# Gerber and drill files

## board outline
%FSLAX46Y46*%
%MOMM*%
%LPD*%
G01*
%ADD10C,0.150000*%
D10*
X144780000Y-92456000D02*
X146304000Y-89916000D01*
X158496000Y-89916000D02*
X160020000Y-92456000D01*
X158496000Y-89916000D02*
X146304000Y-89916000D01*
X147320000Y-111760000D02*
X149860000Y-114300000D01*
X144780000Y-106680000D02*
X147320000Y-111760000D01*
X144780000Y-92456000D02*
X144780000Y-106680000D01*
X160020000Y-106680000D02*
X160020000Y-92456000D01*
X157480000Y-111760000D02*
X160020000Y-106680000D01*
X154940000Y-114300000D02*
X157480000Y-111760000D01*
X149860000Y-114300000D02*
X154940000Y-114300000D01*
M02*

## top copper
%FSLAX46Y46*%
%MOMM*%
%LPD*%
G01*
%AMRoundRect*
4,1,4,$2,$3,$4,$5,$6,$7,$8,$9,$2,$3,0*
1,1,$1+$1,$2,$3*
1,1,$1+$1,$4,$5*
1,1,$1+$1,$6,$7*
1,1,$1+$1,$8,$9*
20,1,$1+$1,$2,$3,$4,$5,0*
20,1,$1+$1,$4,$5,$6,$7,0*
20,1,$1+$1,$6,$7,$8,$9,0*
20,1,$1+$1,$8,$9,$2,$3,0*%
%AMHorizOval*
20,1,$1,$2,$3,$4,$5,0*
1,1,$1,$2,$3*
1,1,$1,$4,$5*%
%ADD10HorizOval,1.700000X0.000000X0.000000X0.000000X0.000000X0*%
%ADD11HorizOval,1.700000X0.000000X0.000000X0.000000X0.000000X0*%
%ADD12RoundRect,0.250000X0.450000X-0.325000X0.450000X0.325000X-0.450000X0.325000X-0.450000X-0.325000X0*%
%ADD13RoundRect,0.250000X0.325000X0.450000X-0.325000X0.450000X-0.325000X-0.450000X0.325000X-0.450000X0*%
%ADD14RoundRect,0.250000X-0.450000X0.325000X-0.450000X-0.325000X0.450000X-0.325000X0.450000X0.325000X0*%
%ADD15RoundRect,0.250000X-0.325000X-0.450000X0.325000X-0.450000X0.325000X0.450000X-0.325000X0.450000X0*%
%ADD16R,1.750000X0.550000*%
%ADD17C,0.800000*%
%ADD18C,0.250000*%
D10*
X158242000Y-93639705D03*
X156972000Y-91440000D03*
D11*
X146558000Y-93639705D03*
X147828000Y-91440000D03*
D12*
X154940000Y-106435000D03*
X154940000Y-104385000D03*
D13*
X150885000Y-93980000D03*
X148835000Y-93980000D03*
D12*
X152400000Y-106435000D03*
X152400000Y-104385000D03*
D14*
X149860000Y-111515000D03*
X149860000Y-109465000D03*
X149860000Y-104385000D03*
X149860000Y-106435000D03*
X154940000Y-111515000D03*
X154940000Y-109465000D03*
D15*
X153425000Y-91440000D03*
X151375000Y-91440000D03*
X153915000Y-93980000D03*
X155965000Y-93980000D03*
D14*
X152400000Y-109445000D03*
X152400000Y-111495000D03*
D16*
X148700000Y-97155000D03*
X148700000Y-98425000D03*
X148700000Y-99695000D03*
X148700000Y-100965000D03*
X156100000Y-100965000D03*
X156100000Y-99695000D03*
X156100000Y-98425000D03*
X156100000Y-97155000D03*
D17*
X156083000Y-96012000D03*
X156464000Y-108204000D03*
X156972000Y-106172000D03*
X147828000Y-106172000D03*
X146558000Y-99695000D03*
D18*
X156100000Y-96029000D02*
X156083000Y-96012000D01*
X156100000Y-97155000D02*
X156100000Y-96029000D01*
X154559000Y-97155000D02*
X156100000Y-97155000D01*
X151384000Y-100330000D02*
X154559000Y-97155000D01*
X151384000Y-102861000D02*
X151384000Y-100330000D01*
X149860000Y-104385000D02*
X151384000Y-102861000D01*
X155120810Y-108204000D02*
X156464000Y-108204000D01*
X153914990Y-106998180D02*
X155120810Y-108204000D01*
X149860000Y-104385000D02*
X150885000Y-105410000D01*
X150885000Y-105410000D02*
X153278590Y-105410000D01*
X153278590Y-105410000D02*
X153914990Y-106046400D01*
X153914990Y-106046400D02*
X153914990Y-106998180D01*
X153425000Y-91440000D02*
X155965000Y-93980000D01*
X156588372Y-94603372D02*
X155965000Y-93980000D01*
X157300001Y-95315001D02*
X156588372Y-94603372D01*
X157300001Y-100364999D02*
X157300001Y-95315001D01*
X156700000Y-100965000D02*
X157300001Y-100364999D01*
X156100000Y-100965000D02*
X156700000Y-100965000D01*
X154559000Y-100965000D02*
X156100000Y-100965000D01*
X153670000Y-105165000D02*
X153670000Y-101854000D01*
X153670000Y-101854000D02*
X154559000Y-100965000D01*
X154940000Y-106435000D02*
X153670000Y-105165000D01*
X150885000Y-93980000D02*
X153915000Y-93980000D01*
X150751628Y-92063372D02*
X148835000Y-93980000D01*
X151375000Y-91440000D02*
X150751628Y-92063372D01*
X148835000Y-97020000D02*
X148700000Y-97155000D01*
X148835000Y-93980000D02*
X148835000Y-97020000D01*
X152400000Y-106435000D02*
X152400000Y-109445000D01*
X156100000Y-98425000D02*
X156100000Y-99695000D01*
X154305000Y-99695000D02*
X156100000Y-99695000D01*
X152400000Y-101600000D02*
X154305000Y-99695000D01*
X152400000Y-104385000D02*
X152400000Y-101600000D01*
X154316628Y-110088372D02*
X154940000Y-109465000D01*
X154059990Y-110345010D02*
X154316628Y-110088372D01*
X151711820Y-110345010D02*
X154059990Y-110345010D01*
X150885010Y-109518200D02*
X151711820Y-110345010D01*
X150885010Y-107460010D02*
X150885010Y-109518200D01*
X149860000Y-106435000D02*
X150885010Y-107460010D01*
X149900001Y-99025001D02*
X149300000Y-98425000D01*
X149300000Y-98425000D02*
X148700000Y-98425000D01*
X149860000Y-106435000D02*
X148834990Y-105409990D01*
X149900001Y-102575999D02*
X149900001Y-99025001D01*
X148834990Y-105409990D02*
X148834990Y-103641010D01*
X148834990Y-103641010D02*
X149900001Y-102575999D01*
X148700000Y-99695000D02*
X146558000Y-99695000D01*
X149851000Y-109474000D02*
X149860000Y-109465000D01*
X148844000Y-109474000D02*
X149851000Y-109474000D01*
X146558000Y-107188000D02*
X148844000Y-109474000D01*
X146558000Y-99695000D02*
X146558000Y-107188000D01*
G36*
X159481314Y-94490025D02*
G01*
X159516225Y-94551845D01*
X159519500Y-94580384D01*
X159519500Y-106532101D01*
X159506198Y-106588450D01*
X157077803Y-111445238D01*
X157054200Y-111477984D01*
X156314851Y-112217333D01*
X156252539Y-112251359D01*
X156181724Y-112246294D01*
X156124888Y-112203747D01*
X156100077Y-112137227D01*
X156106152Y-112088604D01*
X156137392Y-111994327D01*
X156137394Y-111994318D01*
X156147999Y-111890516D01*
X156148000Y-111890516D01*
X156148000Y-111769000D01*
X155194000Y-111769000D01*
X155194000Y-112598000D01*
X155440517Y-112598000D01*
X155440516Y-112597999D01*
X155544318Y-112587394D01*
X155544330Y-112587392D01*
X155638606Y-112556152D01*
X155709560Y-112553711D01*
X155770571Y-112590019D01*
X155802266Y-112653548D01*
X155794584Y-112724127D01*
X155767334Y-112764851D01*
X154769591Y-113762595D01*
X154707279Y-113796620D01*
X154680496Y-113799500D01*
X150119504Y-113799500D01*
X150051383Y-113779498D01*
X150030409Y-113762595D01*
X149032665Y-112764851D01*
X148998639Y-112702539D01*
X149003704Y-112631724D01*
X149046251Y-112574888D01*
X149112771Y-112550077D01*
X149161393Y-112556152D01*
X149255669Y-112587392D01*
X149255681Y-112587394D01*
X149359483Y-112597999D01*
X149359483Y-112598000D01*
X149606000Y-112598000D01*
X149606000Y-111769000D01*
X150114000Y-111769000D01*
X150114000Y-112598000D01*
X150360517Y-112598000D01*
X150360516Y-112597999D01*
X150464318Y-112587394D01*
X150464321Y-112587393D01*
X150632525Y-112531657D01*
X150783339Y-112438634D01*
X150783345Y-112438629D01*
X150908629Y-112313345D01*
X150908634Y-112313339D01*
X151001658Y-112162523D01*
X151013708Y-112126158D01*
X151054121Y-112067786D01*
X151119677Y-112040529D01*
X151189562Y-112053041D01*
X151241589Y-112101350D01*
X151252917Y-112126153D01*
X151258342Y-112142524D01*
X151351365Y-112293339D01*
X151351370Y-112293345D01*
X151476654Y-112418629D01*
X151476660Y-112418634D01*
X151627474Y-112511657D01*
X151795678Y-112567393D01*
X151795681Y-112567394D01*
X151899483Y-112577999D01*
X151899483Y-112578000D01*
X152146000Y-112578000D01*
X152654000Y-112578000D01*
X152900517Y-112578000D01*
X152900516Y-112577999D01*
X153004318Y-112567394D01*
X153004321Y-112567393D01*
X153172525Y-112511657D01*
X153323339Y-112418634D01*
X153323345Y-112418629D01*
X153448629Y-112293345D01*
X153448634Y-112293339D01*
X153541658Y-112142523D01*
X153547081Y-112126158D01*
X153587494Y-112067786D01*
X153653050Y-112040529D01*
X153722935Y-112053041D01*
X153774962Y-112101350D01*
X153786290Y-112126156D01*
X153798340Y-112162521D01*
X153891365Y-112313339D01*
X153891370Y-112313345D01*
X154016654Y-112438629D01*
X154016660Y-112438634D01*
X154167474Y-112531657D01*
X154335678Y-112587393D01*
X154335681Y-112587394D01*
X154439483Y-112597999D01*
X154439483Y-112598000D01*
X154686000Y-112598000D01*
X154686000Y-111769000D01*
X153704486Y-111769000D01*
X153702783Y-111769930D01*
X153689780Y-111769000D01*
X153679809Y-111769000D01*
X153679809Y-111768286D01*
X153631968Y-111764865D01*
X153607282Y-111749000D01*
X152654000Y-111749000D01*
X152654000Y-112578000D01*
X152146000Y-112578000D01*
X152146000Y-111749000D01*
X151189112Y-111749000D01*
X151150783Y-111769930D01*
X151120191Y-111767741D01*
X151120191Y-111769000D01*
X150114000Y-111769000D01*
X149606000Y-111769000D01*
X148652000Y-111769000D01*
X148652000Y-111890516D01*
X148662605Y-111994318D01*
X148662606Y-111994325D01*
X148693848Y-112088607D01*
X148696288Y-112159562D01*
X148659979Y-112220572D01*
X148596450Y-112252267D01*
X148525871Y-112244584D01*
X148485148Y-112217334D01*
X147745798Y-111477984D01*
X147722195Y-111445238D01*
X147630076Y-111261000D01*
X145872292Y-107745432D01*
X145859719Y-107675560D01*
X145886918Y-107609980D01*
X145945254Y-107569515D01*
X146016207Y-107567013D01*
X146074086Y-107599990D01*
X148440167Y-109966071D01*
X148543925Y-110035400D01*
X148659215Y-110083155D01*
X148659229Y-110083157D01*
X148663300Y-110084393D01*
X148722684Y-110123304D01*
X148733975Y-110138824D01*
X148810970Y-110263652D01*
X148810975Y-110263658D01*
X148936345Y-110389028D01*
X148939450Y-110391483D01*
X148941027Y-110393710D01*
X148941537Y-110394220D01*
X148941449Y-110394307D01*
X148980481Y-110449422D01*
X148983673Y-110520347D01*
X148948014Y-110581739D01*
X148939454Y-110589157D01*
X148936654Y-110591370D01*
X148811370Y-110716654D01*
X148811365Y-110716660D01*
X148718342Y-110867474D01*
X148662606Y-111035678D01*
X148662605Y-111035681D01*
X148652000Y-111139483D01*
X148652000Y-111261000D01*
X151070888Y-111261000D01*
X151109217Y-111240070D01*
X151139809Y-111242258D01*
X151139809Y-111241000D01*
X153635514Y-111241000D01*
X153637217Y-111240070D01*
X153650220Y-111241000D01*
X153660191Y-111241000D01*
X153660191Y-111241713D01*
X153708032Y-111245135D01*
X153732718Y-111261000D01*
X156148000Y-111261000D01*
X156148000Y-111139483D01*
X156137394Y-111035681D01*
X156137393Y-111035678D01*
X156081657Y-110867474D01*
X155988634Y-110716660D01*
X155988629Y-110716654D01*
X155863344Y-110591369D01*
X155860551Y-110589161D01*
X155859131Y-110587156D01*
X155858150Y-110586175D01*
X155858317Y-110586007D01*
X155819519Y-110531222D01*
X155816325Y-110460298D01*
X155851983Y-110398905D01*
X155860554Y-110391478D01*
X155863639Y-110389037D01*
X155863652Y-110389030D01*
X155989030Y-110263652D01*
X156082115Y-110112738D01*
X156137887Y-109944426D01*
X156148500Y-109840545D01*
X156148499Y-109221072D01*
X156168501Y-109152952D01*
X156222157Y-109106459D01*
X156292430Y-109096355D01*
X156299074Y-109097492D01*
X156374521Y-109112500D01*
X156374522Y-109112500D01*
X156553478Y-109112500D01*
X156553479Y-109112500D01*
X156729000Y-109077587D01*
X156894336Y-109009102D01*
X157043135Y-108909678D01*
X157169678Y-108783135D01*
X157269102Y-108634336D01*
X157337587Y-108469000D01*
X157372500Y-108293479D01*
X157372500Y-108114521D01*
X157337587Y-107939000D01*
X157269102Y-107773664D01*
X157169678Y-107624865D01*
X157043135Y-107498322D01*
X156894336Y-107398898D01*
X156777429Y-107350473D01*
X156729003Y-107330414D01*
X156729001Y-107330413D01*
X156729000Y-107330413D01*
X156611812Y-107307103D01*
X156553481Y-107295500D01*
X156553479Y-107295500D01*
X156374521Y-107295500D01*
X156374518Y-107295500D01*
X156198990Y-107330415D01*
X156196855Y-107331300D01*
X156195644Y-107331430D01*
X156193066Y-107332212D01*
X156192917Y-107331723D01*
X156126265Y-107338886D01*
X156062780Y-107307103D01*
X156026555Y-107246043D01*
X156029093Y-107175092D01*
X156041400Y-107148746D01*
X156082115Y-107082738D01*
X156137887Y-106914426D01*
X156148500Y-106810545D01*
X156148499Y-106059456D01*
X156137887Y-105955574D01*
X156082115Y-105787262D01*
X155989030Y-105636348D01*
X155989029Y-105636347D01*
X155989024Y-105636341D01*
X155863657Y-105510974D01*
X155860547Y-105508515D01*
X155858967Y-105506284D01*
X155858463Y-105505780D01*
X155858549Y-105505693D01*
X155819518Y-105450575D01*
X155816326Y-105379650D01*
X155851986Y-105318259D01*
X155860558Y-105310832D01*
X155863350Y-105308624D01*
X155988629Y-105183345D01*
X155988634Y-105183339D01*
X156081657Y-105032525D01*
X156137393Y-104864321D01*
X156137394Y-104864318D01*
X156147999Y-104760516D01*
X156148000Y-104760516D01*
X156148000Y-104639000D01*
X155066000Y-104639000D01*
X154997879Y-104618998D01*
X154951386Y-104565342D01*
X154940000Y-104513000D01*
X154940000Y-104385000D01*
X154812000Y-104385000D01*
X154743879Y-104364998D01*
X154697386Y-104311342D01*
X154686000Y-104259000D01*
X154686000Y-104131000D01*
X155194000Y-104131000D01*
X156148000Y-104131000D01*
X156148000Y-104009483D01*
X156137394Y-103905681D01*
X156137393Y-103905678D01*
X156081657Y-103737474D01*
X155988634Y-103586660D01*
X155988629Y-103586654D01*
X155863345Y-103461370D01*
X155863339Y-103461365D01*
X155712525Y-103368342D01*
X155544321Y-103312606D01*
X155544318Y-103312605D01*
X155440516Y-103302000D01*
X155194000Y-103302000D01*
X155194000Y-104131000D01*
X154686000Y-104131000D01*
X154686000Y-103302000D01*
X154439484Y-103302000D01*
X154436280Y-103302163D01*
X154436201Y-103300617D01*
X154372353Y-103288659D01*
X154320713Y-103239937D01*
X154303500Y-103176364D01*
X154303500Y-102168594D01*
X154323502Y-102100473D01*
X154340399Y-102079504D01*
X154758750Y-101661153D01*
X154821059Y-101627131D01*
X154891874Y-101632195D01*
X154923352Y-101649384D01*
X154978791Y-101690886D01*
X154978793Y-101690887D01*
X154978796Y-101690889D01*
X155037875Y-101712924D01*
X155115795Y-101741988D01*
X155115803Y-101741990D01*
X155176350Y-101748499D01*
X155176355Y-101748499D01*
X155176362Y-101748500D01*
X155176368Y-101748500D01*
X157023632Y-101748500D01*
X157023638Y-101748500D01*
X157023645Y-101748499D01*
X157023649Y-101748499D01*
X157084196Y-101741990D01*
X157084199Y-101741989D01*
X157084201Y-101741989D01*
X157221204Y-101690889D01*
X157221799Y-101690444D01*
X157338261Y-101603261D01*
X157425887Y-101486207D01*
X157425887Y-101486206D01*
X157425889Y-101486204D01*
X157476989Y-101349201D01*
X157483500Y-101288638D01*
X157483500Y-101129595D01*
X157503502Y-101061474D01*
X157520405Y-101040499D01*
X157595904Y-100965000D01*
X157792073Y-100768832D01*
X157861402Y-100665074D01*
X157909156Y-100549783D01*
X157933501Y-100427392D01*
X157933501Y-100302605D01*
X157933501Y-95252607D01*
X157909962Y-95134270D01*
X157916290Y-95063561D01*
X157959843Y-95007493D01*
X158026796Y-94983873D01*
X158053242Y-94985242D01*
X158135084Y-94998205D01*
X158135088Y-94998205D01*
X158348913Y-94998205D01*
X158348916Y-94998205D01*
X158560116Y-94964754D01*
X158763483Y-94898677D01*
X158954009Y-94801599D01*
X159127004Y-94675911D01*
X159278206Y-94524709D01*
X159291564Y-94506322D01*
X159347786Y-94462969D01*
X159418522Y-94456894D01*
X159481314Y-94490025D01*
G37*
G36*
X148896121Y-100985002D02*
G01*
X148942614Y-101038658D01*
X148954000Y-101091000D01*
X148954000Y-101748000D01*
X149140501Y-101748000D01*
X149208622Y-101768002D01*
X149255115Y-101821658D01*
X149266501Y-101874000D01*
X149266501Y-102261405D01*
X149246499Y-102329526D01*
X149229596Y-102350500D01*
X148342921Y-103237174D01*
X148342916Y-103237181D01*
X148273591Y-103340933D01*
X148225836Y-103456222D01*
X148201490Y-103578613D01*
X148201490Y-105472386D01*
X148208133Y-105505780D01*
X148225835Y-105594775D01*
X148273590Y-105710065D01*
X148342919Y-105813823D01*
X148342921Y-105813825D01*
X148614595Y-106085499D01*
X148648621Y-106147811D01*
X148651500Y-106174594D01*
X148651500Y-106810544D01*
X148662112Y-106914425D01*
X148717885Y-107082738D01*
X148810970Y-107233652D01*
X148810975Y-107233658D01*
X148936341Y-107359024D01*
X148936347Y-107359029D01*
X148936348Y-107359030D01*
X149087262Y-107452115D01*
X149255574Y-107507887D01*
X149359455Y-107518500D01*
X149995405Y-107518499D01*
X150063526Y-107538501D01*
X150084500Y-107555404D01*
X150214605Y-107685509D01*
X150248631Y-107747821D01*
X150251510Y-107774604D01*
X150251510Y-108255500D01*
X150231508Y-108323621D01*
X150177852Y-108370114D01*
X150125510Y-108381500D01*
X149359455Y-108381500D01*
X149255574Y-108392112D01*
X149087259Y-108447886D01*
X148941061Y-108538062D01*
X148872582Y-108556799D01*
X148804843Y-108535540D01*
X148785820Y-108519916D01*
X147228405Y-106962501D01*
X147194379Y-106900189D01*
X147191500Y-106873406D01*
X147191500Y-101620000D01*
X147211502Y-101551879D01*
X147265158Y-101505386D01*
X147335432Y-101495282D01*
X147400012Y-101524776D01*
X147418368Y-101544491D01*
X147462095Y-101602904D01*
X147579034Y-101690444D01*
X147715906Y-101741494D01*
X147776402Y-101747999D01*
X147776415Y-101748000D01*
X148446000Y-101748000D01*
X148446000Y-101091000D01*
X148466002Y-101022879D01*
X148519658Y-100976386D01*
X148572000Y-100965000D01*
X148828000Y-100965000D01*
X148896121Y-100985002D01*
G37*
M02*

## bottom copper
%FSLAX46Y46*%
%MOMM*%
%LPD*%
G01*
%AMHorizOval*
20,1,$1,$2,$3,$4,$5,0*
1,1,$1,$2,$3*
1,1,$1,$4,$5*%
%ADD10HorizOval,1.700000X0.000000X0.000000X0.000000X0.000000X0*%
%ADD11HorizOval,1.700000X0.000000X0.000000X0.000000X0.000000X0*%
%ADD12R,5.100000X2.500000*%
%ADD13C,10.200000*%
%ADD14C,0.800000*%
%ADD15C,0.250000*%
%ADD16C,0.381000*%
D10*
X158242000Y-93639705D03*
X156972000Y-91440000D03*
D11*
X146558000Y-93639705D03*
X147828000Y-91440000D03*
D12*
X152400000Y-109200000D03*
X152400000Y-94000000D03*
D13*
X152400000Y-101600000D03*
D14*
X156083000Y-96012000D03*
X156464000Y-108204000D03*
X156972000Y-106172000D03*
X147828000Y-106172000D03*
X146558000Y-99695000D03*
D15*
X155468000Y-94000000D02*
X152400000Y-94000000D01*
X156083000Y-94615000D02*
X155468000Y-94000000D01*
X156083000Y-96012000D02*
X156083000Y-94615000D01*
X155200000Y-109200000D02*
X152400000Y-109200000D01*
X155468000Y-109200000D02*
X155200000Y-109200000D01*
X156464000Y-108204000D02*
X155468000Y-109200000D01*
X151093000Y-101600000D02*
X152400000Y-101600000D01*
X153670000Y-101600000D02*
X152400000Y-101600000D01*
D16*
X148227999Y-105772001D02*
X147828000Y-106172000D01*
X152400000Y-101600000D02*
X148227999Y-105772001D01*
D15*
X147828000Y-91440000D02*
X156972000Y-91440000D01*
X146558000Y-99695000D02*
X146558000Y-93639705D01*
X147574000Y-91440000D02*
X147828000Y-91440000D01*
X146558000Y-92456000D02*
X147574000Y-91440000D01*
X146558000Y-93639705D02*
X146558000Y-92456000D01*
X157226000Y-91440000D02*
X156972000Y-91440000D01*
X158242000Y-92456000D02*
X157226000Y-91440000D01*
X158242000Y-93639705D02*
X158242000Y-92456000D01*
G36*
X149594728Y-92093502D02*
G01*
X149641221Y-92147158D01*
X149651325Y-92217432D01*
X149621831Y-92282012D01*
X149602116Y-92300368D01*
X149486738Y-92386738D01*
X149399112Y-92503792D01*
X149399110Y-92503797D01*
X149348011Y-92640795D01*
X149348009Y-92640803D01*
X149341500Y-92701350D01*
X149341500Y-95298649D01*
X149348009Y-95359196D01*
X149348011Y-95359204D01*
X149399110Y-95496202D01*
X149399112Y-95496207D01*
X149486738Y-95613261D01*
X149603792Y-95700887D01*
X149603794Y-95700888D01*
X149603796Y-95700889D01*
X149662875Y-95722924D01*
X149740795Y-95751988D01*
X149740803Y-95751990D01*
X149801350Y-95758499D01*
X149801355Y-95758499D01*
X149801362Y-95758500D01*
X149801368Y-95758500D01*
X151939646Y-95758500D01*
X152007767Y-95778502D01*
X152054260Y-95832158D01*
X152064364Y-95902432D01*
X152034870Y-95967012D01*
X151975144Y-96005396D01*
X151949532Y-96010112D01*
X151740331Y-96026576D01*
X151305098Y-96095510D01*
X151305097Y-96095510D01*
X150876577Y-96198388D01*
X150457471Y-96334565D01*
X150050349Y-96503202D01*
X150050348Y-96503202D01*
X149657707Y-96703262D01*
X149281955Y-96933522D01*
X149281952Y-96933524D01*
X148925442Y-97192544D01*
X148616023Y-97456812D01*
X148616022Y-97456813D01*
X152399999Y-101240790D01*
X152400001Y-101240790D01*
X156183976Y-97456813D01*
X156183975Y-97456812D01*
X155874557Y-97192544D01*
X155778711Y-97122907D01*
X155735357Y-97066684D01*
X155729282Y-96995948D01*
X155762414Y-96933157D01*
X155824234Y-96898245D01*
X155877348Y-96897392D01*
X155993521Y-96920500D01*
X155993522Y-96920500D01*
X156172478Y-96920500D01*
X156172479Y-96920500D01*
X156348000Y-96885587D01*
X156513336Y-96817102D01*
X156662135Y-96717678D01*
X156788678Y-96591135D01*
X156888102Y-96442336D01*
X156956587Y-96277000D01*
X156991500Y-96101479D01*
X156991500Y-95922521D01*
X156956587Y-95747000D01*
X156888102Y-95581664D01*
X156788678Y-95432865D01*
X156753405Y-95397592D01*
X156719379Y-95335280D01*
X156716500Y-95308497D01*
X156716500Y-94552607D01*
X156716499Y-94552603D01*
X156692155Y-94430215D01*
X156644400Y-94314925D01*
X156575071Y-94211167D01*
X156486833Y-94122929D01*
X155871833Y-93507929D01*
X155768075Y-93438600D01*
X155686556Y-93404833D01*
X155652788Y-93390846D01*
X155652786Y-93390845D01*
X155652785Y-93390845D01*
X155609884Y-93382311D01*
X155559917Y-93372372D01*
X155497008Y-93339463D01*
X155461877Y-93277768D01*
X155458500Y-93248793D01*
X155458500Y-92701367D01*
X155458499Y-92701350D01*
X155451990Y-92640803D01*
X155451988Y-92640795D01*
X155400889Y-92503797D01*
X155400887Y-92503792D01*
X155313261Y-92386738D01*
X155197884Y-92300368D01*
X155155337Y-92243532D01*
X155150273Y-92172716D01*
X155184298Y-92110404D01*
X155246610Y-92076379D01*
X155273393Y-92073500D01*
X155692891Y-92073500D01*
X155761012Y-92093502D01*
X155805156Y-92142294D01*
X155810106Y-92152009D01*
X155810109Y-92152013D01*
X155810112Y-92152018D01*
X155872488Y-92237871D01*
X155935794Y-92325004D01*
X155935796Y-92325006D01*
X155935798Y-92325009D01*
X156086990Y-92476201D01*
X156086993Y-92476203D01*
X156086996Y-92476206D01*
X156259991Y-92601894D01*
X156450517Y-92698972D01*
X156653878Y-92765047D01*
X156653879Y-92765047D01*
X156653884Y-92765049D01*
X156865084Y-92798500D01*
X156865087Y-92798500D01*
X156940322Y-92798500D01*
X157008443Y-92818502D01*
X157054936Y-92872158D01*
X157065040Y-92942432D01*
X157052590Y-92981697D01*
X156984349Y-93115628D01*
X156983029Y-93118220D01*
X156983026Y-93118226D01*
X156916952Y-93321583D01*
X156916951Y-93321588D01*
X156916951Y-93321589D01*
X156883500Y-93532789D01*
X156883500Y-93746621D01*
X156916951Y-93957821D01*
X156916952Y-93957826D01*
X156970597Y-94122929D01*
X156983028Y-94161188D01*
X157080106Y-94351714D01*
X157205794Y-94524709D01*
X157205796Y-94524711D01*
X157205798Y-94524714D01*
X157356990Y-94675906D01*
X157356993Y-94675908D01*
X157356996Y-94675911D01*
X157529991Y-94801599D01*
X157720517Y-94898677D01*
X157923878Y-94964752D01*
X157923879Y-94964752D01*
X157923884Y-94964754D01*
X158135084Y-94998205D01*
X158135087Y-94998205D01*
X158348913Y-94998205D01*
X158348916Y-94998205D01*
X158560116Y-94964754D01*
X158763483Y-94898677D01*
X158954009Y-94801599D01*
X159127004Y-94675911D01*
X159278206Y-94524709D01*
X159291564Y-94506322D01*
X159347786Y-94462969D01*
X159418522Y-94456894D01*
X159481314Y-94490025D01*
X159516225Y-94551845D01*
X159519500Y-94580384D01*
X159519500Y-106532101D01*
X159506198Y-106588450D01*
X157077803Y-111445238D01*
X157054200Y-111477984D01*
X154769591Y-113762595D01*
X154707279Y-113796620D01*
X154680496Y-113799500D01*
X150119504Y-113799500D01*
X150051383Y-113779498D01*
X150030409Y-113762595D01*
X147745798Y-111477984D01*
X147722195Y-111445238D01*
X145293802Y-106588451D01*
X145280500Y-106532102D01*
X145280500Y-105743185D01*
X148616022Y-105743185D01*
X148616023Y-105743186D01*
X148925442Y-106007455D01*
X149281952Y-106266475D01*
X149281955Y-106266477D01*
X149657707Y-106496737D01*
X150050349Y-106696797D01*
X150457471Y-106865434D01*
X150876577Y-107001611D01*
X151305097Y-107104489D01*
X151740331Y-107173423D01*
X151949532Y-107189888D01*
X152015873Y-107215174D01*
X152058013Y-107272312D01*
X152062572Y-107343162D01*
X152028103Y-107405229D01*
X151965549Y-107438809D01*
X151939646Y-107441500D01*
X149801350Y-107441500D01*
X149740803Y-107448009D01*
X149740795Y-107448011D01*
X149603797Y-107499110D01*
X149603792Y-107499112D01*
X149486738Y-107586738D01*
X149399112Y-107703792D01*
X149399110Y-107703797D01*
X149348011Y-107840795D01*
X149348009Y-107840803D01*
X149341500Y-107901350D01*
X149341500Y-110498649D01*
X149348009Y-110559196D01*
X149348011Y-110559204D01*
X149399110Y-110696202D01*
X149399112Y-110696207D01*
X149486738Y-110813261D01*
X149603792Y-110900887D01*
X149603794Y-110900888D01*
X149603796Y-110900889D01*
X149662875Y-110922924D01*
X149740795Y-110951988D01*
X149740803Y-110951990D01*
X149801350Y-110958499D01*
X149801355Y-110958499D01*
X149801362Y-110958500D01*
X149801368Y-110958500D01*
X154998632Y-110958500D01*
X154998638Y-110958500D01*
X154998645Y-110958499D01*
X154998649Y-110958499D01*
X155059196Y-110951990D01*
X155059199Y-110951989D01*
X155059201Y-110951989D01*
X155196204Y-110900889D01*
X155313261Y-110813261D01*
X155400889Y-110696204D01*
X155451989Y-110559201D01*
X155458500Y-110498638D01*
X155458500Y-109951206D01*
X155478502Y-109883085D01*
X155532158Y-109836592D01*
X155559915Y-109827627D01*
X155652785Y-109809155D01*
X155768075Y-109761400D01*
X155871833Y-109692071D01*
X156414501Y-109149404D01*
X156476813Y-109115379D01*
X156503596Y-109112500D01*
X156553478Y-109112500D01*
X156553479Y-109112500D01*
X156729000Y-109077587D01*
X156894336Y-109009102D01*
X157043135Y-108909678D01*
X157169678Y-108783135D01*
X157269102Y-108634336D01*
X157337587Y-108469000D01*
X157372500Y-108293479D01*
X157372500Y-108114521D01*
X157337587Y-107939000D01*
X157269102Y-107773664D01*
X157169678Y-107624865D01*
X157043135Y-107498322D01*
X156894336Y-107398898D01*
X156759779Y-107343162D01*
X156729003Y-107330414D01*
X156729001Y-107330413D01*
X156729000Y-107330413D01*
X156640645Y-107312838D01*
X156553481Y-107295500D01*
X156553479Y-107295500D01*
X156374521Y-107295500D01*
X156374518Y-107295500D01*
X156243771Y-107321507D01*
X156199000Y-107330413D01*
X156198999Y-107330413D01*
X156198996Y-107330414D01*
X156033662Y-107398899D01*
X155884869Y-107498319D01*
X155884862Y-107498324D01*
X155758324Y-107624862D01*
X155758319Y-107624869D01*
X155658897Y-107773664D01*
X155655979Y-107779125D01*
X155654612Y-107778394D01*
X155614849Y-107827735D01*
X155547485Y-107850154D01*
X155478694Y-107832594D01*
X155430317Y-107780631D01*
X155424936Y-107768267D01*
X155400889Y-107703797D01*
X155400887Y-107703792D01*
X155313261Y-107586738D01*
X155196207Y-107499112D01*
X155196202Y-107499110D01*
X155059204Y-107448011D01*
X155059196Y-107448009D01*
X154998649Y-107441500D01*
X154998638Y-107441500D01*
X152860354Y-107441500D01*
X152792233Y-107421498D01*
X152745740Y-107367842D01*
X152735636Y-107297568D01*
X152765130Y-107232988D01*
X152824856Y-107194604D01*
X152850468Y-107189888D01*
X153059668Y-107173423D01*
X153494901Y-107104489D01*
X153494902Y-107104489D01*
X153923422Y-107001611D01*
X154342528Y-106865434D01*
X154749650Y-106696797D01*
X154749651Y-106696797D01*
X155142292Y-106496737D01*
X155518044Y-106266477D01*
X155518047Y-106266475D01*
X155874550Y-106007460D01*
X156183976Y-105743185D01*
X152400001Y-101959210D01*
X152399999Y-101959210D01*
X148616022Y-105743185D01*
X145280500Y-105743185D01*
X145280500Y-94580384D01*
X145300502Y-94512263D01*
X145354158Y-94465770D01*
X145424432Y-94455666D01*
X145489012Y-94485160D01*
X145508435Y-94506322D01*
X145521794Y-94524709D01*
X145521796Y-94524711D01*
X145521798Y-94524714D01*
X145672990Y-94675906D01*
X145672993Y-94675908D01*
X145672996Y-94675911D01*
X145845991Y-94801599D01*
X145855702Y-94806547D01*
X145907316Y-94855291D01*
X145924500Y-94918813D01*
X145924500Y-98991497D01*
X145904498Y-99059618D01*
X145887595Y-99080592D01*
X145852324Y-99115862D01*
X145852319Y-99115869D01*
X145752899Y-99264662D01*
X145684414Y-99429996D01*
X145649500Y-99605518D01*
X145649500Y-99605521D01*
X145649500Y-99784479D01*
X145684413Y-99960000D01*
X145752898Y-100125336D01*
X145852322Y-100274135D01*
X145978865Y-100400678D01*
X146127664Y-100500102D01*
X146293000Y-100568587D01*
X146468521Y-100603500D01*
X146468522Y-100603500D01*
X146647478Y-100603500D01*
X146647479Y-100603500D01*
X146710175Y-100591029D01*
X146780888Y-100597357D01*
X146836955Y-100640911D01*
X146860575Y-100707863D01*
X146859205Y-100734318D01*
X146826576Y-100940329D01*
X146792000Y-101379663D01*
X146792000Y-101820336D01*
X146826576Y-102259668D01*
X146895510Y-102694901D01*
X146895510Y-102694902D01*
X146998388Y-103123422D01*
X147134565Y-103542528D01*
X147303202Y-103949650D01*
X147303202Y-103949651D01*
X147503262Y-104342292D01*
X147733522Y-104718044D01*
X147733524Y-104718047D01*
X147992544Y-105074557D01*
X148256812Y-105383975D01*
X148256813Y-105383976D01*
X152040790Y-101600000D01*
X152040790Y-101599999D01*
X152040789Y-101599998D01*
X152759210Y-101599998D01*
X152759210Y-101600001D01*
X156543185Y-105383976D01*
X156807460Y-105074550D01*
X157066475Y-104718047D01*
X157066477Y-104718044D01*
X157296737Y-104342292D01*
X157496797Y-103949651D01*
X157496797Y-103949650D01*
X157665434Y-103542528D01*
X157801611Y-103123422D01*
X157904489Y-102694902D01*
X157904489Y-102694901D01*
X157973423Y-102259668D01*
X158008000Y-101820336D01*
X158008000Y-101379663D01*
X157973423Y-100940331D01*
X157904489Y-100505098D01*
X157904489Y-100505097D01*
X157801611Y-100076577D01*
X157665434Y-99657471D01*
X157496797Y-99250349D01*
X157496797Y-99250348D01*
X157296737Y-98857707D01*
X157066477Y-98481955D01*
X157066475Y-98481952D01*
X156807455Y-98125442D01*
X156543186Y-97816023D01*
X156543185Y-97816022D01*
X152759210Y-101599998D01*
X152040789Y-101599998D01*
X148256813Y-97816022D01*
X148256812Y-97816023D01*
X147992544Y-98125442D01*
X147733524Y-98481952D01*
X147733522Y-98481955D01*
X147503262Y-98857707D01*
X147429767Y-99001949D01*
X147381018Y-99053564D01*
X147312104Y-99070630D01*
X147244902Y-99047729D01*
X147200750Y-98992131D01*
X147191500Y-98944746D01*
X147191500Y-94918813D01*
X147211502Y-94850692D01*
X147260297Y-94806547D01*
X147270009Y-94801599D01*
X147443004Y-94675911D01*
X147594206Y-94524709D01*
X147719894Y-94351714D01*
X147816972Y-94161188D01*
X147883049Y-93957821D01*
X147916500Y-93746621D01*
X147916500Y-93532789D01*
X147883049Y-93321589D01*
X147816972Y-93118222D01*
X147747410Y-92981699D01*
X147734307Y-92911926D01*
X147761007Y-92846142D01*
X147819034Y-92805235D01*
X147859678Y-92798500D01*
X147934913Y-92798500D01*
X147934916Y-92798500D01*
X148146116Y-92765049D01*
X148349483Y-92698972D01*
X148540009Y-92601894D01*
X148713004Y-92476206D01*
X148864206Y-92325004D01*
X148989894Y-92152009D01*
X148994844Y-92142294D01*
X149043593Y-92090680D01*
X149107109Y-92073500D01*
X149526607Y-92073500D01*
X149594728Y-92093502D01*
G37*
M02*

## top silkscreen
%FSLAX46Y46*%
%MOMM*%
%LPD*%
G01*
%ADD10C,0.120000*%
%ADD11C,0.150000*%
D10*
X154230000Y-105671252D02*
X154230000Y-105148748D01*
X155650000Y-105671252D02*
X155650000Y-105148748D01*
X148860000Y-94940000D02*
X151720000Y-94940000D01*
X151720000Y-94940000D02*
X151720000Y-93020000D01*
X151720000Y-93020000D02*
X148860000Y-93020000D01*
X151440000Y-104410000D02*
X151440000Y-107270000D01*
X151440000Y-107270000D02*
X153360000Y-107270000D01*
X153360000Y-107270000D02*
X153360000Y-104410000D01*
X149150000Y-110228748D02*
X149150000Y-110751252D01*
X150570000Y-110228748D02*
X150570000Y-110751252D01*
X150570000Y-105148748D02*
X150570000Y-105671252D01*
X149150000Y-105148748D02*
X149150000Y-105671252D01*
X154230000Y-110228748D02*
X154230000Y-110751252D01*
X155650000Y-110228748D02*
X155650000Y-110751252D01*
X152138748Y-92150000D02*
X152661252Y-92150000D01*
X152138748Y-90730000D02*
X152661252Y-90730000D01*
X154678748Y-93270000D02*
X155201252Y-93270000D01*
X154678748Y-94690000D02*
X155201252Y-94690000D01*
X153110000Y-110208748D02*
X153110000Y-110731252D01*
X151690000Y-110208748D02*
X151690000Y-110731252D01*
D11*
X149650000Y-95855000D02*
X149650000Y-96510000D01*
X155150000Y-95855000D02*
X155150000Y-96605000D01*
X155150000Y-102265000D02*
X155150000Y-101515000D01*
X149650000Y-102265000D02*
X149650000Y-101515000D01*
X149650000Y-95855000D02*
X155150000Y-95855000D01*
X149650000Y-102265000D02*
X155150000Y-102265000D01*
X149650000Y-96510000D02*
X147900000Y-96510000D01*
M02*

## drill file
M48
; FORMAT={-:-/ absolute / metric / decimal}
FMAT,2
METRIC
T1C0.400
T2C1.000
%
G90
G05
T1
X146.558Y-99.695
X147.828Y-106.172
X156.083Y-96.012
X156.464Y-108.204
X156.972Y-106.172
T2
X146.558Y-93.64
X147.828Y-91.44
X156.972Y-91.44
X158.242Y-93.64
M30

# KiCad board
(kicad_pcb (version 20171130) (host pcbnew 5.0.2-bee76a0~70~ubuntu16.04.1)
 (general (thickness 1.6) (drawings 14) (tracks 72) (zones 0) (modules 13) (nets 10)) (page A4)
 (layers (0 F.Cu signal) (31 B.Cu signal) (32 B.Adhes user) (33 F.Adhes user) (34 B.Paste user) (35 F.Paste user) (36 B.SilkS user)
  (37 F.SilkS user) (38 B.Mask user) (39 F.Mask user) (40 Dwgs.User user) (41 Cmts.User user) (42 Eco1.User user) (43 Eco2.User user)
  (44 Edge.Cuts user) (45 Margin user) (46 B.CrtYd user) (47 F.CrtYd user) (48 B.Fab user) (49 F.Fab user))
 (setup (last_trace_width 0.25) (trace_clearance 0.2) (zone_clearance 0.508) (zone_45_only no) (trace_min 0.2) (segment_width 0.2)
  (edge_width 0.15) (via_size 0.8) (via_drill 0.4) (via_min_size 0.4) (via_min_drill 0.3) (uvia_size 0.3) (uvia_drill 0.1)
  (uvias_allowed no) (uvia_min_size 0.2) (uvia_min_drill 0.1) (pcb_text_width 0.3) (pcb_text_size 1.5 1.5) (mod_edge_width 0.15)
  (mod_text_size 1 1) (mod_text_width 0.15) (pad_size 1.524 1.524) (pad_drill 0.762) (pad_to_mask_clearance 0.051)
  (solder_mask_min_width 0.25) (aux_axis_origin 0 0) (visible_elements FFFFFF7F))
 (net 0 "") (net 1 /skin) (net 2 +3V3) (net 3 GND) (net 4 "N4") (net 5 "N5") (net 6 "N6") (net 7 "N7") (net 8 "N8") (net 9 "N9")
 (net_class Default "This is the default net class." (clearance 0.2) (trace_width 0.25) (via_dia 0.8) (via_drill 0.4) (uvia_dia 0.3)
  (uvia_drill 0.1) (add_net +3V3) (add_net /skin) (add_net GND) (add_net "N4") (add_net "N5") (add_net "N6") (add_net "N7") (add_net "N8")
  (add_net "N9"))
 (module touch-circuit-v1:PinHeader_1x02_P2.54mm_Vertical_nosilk (layer F.Cu) (at 156.972 91.44 30)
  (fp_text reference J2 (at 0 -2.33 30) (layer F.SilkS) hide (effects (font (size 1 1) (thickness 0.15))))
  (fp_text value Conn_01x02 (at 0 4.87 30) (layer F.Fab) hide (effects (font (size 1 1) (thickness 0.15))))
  (pad 2 thru_hole oval (at 0 2.54 30) (size 1.7 1.7) (drill 1) (layers *.Cu *.Mask) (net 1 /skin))
  (pad 1 thru_hole oval (at 0 0 30) (size 1.7 1.7) (drill 1) (layers *.Cu *.Mask) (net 1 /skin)))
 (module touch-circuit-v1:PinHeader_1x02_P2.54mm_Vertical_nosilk (layer F.Cu) (at 147.828 91.44 330)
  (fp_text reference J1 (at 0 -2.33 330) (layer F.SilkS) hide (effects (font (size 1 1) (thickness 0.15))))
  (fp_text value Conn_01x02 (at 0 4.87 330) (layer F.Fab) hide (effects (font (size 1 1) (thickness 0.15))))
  (pad 2 thru_hole oval (at 0 2.54 330) (size 1.7 1.7) (drill 1) (layers *.Cu *.Mask) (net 1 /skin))
  (pad 1 thru_hole oval (at 0 0 330) (size 1.7 1.7) (drill 1) (layers *.Cu *.Mask) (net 1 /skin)))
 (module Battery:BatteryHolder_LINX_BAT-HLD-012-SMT (layer B.Cu) (at 152.4 101.6 90)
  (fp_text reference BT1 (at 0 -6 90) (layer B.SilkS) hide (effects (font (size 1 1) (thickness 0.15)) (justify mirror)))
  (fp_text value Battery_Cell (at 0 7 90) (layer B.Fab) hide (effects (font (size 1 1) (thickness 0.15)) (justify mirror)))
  (pad 1 smd rect (at -7.6 0 90) (size 2.5 5.1) (layers B.Cu B.Paste B.Mask) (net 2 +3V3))
  (pad 1 smd rect (at 7.6 0 90) (size 2.5 5.1) (layers B.Cu B.Paste B.Mask) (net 2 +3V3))
  (pad 2 smd circle (at 0 0 90) (size 10.2 10.2) (layers B.Cu B.Paste B.Mask) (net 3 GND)))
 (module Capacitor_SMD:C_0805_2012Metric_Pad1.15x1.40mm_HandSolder (layer F.Cu) (at 154.94 105.41 90)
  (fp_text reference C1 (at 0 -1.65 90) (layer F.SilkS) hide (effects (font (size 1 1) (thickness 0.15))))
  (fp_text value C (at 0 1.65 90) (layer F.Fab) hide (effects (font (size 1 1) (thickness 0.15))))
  (fp_line (start -0.261252 -0.71) (end 0.261252 -0.71) (layer F.SilkS) (width 0.12))
  (fp_line (start -0.261252 0.71) (end 0.261252 0.71) (layer F.SilkS) (width 0.12))
  (pad 1 smd roundrect (at -1.025 0 90) (size 1.15 1.4) (layers F.Cu F.Paste F.Mask) (roundrect_rratio 0.217391) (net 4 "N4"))
  (pad 2 smd roundrect (at 1.025 0 90) (size 1.15 1.4) (layers F.Cu F.Paste F.Mask) (roundrect_rratio 0.217391) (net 3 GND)))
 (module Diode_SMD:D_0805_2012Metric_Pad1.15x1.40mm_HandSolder (layer F.Cu) (at 149.86 93.98 180)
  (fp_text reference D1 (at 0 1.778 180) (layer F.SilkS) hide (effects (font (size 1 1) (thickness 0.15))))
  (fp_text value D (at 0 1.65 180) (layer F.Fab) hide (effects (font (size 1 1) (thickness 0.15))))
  (fp_line (start 1 -0.96) (end -1.86 -0.96) (layer F.SilkS) (width 0.12))
  (fp_line (start -1.86 -0.96) (end -1.86 0.96) (layer F.SilkS) (width 0.12))
  (fp_line (start -1.86 0.96) (end 1 0.96) (layer F.SilkS) (width 0.12))
  (pad 1 smd roundrect (at -1.025 0 180) (size 1.15 1.4) (layers F.Cu F.Paste F.Mask) (roundrect_rratio 0.217391) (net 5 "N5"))
  (pad 2 smd roundrect (at 1.025 0 180) (size 1.15 1.4) (layers F.Cu F.Paste F.Mask) (roundrect_rratio 0.217391) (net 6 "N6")))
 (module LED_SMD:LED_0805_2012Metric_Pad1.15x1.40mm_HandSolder (layer F.Cu) (at 152.4 105.41 90)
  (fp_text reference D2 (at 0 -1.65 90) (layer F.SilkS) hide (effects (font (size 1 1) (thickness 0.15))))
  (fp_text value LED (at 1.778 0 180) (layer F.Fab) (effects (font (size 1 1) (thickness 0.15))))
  (fp_line (start 1 -0.96) (end -1.86 -0.96) (layer F.SilkS) (width 0.12))
  (fp_line (start -1.86 -0.96) (end -1.86 0.96) (layer F.SilkS) (width 0.12))
  (fp_line (start -1.86 0.96) (end 1 0.96) (layer F.SilkS) (width 0.12))
  (pad 1 smd roundrect (at -1.025 0 90) (size 1.15 1.4) (layers F.Cu F.Paste F.Mask) (roundrect_rratio 0.217391) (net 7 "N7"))
  (pad 2 smd roundrect (at 1.025 0 90) (size 1.15 1.4) (layers F.Cu F.Paste F.Mask) (roundrect_rratio 0.217391) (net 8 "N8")))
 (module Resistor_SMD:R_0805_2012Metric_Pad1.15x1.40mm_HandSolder (layer F.Cu) (at 149.86 110.49 270)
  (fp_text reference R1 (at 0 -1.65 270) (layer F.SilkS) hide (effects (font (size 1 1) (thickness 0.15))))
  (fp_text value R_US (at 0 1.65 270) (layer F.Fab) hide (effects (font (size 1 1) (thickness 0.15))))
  (fp_line (start -0.261252 0.71) (end 0.261252 0.71) (layer F.SilkS) (width 0.12))
  (fp_line (start -0.261252 -0.71) (end 0.261252 -0.71) (layer F.SilkS) (width 0.12))
  (pad 2 smd roundrect (at 1.025 0 270) (size 1.15 1.4) (layers F.Cu F.Paste F.Mask) (roundrect_rratio 0.217391) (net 3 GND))
  (pad 1 smd roundrect (at -1.025 0 270) (size 1.15 1.4) (layers F.Cu F.Paste F.Mask) (roundrect_rratio 0.217391) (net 1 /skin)))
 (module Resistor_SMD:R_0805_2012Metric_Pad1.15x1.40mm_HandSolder (layer F.Cu) (at 149.86 105.41 270)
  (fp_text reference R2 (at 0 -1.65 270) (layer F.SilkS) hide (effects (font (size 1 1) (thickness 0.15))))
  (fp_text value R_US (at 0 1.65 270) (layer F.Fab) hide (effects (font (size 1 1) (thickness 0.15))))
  (fp_line (start -0.261252 -0.71) (end 0.261252 -0.71) (layer F.SilkS) (width 0.12))
  (fp_line (start -0.261252 0.71) (end 0.261252 0.71) (layer F.SilkS) (width 0.12))
  (pad 1 smd roundrect (at -1.025 0 270) (size 1.15 1.4) (layers F.Cu F.Paste F.Mask) (roundrect_rratio 0.217391) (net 2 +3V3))
  (pad 2 smd roundrect (at 1.025 0 270) (size 1.15 1.4) (layers F.Cu F.Paste F.Mask) (roundrect_rratio 0.217391) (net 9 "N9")))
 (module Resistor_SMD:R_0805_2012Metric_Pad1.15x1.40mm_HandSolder (layer F.Cu) (at 154.94 110.49 270)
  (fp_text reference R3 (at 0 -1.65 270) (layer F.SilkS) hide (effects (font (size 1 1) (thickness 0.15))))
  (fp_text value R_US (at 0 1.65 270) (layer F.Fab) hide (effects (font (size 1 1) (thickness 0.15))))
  (fp_line (start -0.261252 0.71) (end 0.261252 0.71) (layer F.SilkS) (width 0.12))
  (fp_line (start -0.261252 -0.71) (end 0.261252 -0.71) (layer F.SilkS) (width 0.12))
  (pad 2 smd roundrect (at 1.025 0 270) (size 1.15 1.4) (layers F.Cu F.Paste F.Mask) (roundrect_rratio 0.217391) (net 3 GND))
  (pad 1 smd roundrect (at -1.025 0 270) (size 1.15 1.4) (layers F.Cu F.Paste F.Mask) (roundrect_rratio 0.217391) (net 9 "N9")))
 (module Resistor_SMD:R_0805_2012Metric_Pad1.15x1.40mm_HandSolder (layer F.Cu) (at 152.4 91.44)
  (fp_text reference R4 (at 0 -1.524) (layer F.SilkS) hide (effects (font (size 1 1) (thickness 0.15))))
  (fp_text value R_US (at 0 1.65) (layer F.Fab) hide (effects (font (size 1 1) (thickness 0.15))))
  (fp_line (start -0.261252 0.71) (end 0.261252 0.71) (layer F.SilkS) (width 0.12))
  (fp_line (start -0.261252 -0.71) (end 0.261252 -0.71) (layer F.SilkS) (width 0.12))
  (pad 2 smd roundrect (at 1.025 0) (size 1.15 1.4) (layers F.Cu F.Paste F.Mask) (roundrect_rratio 0.217391) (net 4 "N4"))
  (pad 1 smd roundrect (at -1.025 0) (size 1.15 1.4) (layers F.Cu F.Paste F.Mask) (roundrect_rratio 0.217391) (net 6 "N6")))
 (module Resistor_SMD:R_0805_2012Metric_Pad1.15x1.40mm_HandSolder (layer F.Cu) (at 154.94 93.98)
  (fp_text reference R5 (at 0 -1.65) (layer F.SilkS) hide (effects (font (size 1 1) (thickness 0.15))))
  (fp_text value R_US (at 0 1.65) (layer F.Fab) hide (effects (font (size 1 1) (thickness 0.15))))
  (fp_line (start -0.261252 -0.71) (end 0.261252 -0.71) (layer F.SilkS) (width 0.12))
  (fp_line (start -0.261252 0.71) (end 0.261252 0.71) (layer F.SilkS) (width 0.12))
  (pad 1 smd roundrect (at -1.025 0) (size 1.15 1.4) (layers F.Cu F.Paste F.Mask) (roundrect_rratio 0.217391) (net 5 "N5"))
  (pad 2 smd roundrect (at 1.025 0) (size 1.15 1.4) (layers F.Cu F.Paste F.Mask) (roundrect_rratio 0.217391) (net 4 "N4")))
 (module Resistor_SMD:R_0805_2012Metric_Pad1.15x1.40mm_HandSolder (layer F.Cu) (at 152.4 110.47 270)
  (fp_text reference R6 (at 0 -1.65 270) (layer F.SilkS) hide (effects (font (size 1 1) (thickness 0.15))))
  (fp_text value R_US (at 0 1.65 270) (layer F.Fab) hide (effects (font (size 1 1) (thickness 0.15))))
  (fp_line (start -0.261252 -0.71) (end 0.261252 -0.71) (layer F.SilkS) (width 0.12))
  (fp_line (start -0.261252 0.71) (end 0.261252 0.71) (layer F.SilkS) (width 0.12))
  (pad 1 smd roundrect (at -1.025 0 270) (size 1.15 1.4) (layers F.Cu F.Paste F.Mask) (roundrect_rratio 0.217391) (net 7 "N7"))
  (pad 2 smd roundrect (at 1.025 0 270) (size 1.15 1.4) (layers F.Cu F.Paste F.Mask) (roundrect_rratio 0.217391) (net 3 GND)))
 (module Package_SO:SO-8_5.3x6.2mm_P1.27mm (layer F.Cu) (at 152.4 99.06)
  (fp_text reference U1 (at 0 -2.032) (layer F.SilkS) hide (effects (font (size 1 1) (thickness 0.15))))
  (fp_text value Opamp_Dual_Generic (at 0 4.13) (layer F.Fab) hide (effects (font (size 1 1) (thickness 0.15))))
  (fp_line (start -2.75 -3.205) (end -2.75 -2.55) (layer F.SilkS) (width 0.15))
  (fp_line (start 2.75 -3.205) (end 2.75 -2.455) (layer F.SilkS) (width 0.15))
  (fp_line (start 2.75 3.205) (end 2.75 2.455) (layer F.SilkS) (width 0.15))
  (fp_line (start -2.75 3.205) (end -2.75 2.455) (layer F.SilkS) (width 0.15))
  (fp_line (start -2.75 -3.205) (end 2.75 -3.205) (layer F.SilkS) (width 0.15))
  (fp_line (start -2.75 3.205) (end 2.75 3.205) (layer F.SilkS) (width 0.15))
  (fp_line (start -2.75 -2.55) (end -4.5 -2.55) (layer F.SilkS) (width 0.15))
  (pad 1 smd rect (at -3.7 -1.905) (size 1.75 0.55) (layers F.Cu F.Paste F.Mask) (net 6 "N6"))
  (pad 2 smd rect (at -3.7 -0.635) (size 1.75 0.55) (layers F.Cu F.Paste F.Mask) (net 9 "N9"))
  (pad 3 smd rect (at -3.7 0.635) (size 1.75 0.55) (layers F.Cu F.Paste F.Mask) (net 1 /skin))
  (pad 4 smd rect (at -3.7 1.905) (size 1.75 0.55) (layers F.Cu F.Paste F.Mask) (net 3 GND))
  (pad 5 smd rect (at 3.7 1.905) (size 1.75 0.55) (layers F.Cu F.Paste F.Mask) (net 4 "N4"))
  (pad 6 smd rect (at 3.7 0.635) (size 1.75 0.55) (layers F.Cu F.Paste F.Mask) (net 8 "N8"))
  (pad 7 smd rect (at 3.7 -0.635) (size 1.75 0.55) (layers F.Cu F.Paste F.Mask) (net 8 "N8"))
  (pad 8 smd rect (at 3.7 -1.905) (size 1.75 0.55) (layers F.Cu F.Paste F.Mask) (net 2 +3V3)))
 (gr_line (start 144.78 92.456) (end 146.304 89.916) (layer Edge.Cuts) (width 0.15))
 (gr_line (start 158.496 89.916) (end 160.02 92.456) (layer Edge.Cuts) (width 0.15))
 (gr_line (start 158.496 89.916) (end 146.304 89.916) (layer Edge.Cuts) (width 0.15))
 (gr_line (start 147.32 111.76) (end 149.86 114.3) (layer Edge.Cuts) (width 0.15))
 (gr_line (start 144.78 106.68) (end 147.32 111.76) (layer Edge.Cuts) (width 0.15))
 (gr_line (start 144.78 92.456) (end 144.78 106.68) (layer Edge.Cuts) (width 0.15))
 (gr_line (start 160.02 106.68) (end 160.02 92.456) (layer Edge.Cuts) (width 0.15))
 (gr_line (start 157.48 111.76) (end 160.02 106.68) (layer Edge.Cuts) (width 0.15))
 (gr_line (start 154.94 114.3) (end 157.48 111.76) (layer Edge.Cuts) (width 0.15))
 (gr_line (start 149.86 114.3) (end 154.94 114.3) (layer Edge.Cuts) (width 0.15))
 (via (at 156.083 96.012) (size 0.8) (drill 0.4) (layers F.Cu B.Cu) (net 2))
 (segment (start 156.1 96.029) (end 156.083 96.012) (width 0.25) (layer F.Cu) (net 2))
 (segment (start 156.1 97.155) (end 156.1 96.029) (width 0.25) (layer F.Cu) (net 2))
 (segment (start 155.468 94) (end 152.4 94) (width 0.25) (layer B.Cu) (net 2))
 (segment (start 156.083 94.615) (end 155.468 94) (width 0.25) (layer B.Cu) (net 2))
 (segment (start 156.083 96.012) (end 156.083 94.615) (width 0.25) (layer B.Cu) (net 2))
 (segment (start 154.559 97.155) (end 156.1 97.155) (width 0.25) (layer F.Cu) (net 2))
 (segment (start 151.384 100.33) (end 154.559 97.155) (width 0.25) (layer F.Cu) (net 2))
 (segment (start 151.384 102.861) (end 151.384 100.33) (width 0.25) (layer F.Cu) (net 2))
 (segment (start 149.86 104.385) (end 151.384 102.861) (width 0.25) (layer F.Cu) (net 2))
 (via (at 156.464 108.204) (size 0.8) (drill 0.4) (layers F.Cu B.Cu) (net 2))
 (segment (start 155.2 109.2) (end 152.4 109.2) (width 0.25) (layer B.Cu) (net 2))
 (segment (start 155.468 109.2) (end 155.2 109.2) (width 0.25) (layer B.Cu) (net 2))
 (segment (start 156.464 108.204) (end 155.468 109.2) (width 0.25) (layer B.Cu) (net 2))
 (segment (start 155.12081 108.204) (end 156.464 108.204) (width 0.25) (layer F.Cu) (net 2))
 (segment (start 153.91499 106.99818) (end 155.12081 108.204) (width 0.25) (layer F.Cu) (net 2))
 (segment (start 149.86 104.385) (end 150.885 105.41) (width 0.25) (layer F.Cu) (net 2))
 (segment (start 150.885 105.41) (end 153.27859 105.41) (width 0.25) (layer F.Cu) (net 2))
 (segment (start 153.27859 105.41) (end 153.91499 106.0464) (width 0.25) (layer F.Cu) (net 2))
 (segment (start 153.91499 106.0464) (end 153.91499 106.99818) (width 0.25) (layer F.Cu) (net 2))
 (segment (start 151.093 101.6) (end 152.4 101.6) (width 0.25) (layer B.Cu) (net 3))
 (via (at 156.972 106.172) (size 0.8) (drill 0.4) (layers F.Cu B.Cu) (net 3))
 (segment (start 153.67 101.6) (end 152.4 101.6) (width 0.25) (layer B.Cu) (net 3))
 (segment (start 148.227999 105.772001) (end 147.828 106.172) (width 0.381) (layer B.Cu) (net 3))
 (segment (start 152.4 101.6) (end 148.227999 105.772001) (width 0.381) (layer B.Cu) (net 3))
 (via (at 147.828 106.172) (size 0.8) (drill 0.4) (layers F.Cu B.Cu) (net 3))
 (segment (start 153.425 91.44) (end 155.965 93.98) (width 0.25) (layer F.Cu) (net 4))
 (segment (start 156.588372 94.603372) (end 155.965 93.98) (width 0.25) (layer F.Cu) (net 4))
 (segment (start 157.300001 95.315001) (end 156.588372 94.603372) (width 0.25) (layer F.Cu) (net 4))
 (segment (start 157.300001 100.364999) (end 157.300001 95.315001) (width 0.25) (layer F.Cu) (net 4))
 (segment (start 156.7 100.965) (end 157.300001 100.364999) (width 0.25) (layer F.Cu) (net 4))
 (segment (start 156.1 100.965) (end 156.7 100.965) (width 0.25) (layer F.Cu) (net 4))
 (segment (start 154.559 100.965) (end 156.1 100.965) (width 0.25) (layer F.Cu) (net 4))
 (segment (start 153.67 105.165) (end 153.67 101.854) (width 0.25) (layer F.Cu) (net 4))
 (segment (start 153.67 101.854) (end 154.559 100.965) (width 0.25) (layer F.Cu) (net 4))
 (segment (start 154.94 106.435) (end 153.67 105.165) (width 0.25) (layer F.Cu) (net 4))
 (segment (start 150.885 93.98) (end 153.915 93.98) (width 0.25) (layer F.Cu) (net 5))
 (segment (start 150.751628 92.063372) (end 148.835 93.98) (width 0.25) (layer F.Cu) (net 6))
 (segment (start 151.375 91.44) (end 150.751628 92.063372) (width 0.25) (layer F.Cu) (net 6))
 (segment (start 148.835 97.02) (end 148.7 97.155) (width 0.25) (layer F.Cu) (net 6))
 (segment (start 148.835 93.98) (end 148.835 97.02) (width 0.25) (layer F.Cu) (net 6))
 (segment (start 152.4 106.435) (end 152.4 109.445) (width 0.25) (layer F.Cu) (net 7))
 (segment (start 156.1 98.425) (end 156.1 99.695) (width 0.25) (layer F.Cu) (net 8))
 (segment (start 154.305 99.695) (end 156.1 99.695) (width 0.25) (layer F.Cu) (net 8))
 (segment (start 152.4 101.6) (end 154.305 99.695) (width 0.25) (layer F.Cu) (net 8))
 (segment (start 152.4 104.385) (end 152.4 101.6) (width 0.25) (layer F.Cu) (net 8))
 (segment (start 154.316628 110.088372) (end 154.94 109.465) (width 0.25) (layer F.Cu) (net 9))
 (segment (start 154.05999 110.34501) (end 154.316628 110.088372) (width 0.25) (layer F.Cu) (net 9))
 (segment (start 151.71182 110.34501) (end 154.05999 110.34501) (width 0.25) (layer F.Cu) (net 9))
 (segment (start 150.88501 109.5182) (end 151.71182 110.34501) (width 0.25) (layer F.Cu) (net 9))
 (segment (start 150.88501 107.46001) (end 150.88501 109.5182) (width 0.25) (layer F.Cu) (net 9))
 (segment (start 149.86 106.435) (end 150.88501 107.46001) (width 0.25) (layer F.Cu) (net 9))
 (segment (start 149.900001 99.025001) (end 149.3 98.425) (width 0.25) (layer F.Cu) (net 9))
 (segment (start 149.3 98.425) (end 148.7 98.425) (width 0.25) (layer F.Cu) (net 9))
 (segment (start 149.86 106.435) (end 148.83499 105.40999) (width 0.25) (layer F.Cu) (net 9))
 (segment (start 149.900001 102.575999) (end 149.900001 99.025001) (width 0.25) (layer F.Cu) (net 9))
 (segment (start 148.83499 105.40999) (end 148.83499 103.64101) (width 0.25) (layer F.Cu) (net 9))
 (segment (start 148.83499 103.64101) (end 149.900001 102.575999) (width 0.25) (layer F.Cu) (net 9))
 (segment (start 147.828 91.44) (end 156.972 91.44) (width 0.25) (layer B.Cu) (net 1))
 (via (at 146.558 99.695) (size 0.8) (drill 0.4) (layers F.Cu B.Cu) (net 1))
 (segment (start 148.7 99.695) (end 146.558 99.695) (width 0.25) (layer F.Cu) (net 1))
 (segment (start 146.558 99.695) (end 146.558 93.639705) (width 0.25) (layer B.Cu) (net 1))
 (segment (start 149.851 109.474) (end 149.86 109.465) (width 0.25) (layer F.Cu) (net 1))
 (segment (start 148.844 109.474) (end 149.851 109.474) (width 0.25) (layer F.Cu) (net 1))
 (segment (start 146.558 107.188) (end 148.844 109.474) (width 0.25) (layer F.Cu) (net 1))
 (segment (start 146.558 99.695) (end 146.558 107.188) (width 0.25) (layer F.Cu) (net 1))
 (segment (start 147.574 91.44) (end 147.828 91.44) (width 0.25) (layer B.Cu) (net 1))
 (segment (start 146.558 92.456) (end 147.574 91.44) (width 0.25) (layer B.Cu) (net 1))
 (segment (start 146.558 93.639705) (end 146.558 92.456) (width 0.25) (layer B.Cu) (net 1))
 (segment (start 157.226 91.44) (end 156.972 91.44) (width 0.25) (layer B.Cu) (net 1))
 (segment (start 158.242 92.456) (end 157.226 91.44) (width 0.25) (layer B.Cu) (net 1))
 (segment (start 158.242 93.639705) (end 158.242 92.456) (width 0.25) (layer B.Cu) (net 1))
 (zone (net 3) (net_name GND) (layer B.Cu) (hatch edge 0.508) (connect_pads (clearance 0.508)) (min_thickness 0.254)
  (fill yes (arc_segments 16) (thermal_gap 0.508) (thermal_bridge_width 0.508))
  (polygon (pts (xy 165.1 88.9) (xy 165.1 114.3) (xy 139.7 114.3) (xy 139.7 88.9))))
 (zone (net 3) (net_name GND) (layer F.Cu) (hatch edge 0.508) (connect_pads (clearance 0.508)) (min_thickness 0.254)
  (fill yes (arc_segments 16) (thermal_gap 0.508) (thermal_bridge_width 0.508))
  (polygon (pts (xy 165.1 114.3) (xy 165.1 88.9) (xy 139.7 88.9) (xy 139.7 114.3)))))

